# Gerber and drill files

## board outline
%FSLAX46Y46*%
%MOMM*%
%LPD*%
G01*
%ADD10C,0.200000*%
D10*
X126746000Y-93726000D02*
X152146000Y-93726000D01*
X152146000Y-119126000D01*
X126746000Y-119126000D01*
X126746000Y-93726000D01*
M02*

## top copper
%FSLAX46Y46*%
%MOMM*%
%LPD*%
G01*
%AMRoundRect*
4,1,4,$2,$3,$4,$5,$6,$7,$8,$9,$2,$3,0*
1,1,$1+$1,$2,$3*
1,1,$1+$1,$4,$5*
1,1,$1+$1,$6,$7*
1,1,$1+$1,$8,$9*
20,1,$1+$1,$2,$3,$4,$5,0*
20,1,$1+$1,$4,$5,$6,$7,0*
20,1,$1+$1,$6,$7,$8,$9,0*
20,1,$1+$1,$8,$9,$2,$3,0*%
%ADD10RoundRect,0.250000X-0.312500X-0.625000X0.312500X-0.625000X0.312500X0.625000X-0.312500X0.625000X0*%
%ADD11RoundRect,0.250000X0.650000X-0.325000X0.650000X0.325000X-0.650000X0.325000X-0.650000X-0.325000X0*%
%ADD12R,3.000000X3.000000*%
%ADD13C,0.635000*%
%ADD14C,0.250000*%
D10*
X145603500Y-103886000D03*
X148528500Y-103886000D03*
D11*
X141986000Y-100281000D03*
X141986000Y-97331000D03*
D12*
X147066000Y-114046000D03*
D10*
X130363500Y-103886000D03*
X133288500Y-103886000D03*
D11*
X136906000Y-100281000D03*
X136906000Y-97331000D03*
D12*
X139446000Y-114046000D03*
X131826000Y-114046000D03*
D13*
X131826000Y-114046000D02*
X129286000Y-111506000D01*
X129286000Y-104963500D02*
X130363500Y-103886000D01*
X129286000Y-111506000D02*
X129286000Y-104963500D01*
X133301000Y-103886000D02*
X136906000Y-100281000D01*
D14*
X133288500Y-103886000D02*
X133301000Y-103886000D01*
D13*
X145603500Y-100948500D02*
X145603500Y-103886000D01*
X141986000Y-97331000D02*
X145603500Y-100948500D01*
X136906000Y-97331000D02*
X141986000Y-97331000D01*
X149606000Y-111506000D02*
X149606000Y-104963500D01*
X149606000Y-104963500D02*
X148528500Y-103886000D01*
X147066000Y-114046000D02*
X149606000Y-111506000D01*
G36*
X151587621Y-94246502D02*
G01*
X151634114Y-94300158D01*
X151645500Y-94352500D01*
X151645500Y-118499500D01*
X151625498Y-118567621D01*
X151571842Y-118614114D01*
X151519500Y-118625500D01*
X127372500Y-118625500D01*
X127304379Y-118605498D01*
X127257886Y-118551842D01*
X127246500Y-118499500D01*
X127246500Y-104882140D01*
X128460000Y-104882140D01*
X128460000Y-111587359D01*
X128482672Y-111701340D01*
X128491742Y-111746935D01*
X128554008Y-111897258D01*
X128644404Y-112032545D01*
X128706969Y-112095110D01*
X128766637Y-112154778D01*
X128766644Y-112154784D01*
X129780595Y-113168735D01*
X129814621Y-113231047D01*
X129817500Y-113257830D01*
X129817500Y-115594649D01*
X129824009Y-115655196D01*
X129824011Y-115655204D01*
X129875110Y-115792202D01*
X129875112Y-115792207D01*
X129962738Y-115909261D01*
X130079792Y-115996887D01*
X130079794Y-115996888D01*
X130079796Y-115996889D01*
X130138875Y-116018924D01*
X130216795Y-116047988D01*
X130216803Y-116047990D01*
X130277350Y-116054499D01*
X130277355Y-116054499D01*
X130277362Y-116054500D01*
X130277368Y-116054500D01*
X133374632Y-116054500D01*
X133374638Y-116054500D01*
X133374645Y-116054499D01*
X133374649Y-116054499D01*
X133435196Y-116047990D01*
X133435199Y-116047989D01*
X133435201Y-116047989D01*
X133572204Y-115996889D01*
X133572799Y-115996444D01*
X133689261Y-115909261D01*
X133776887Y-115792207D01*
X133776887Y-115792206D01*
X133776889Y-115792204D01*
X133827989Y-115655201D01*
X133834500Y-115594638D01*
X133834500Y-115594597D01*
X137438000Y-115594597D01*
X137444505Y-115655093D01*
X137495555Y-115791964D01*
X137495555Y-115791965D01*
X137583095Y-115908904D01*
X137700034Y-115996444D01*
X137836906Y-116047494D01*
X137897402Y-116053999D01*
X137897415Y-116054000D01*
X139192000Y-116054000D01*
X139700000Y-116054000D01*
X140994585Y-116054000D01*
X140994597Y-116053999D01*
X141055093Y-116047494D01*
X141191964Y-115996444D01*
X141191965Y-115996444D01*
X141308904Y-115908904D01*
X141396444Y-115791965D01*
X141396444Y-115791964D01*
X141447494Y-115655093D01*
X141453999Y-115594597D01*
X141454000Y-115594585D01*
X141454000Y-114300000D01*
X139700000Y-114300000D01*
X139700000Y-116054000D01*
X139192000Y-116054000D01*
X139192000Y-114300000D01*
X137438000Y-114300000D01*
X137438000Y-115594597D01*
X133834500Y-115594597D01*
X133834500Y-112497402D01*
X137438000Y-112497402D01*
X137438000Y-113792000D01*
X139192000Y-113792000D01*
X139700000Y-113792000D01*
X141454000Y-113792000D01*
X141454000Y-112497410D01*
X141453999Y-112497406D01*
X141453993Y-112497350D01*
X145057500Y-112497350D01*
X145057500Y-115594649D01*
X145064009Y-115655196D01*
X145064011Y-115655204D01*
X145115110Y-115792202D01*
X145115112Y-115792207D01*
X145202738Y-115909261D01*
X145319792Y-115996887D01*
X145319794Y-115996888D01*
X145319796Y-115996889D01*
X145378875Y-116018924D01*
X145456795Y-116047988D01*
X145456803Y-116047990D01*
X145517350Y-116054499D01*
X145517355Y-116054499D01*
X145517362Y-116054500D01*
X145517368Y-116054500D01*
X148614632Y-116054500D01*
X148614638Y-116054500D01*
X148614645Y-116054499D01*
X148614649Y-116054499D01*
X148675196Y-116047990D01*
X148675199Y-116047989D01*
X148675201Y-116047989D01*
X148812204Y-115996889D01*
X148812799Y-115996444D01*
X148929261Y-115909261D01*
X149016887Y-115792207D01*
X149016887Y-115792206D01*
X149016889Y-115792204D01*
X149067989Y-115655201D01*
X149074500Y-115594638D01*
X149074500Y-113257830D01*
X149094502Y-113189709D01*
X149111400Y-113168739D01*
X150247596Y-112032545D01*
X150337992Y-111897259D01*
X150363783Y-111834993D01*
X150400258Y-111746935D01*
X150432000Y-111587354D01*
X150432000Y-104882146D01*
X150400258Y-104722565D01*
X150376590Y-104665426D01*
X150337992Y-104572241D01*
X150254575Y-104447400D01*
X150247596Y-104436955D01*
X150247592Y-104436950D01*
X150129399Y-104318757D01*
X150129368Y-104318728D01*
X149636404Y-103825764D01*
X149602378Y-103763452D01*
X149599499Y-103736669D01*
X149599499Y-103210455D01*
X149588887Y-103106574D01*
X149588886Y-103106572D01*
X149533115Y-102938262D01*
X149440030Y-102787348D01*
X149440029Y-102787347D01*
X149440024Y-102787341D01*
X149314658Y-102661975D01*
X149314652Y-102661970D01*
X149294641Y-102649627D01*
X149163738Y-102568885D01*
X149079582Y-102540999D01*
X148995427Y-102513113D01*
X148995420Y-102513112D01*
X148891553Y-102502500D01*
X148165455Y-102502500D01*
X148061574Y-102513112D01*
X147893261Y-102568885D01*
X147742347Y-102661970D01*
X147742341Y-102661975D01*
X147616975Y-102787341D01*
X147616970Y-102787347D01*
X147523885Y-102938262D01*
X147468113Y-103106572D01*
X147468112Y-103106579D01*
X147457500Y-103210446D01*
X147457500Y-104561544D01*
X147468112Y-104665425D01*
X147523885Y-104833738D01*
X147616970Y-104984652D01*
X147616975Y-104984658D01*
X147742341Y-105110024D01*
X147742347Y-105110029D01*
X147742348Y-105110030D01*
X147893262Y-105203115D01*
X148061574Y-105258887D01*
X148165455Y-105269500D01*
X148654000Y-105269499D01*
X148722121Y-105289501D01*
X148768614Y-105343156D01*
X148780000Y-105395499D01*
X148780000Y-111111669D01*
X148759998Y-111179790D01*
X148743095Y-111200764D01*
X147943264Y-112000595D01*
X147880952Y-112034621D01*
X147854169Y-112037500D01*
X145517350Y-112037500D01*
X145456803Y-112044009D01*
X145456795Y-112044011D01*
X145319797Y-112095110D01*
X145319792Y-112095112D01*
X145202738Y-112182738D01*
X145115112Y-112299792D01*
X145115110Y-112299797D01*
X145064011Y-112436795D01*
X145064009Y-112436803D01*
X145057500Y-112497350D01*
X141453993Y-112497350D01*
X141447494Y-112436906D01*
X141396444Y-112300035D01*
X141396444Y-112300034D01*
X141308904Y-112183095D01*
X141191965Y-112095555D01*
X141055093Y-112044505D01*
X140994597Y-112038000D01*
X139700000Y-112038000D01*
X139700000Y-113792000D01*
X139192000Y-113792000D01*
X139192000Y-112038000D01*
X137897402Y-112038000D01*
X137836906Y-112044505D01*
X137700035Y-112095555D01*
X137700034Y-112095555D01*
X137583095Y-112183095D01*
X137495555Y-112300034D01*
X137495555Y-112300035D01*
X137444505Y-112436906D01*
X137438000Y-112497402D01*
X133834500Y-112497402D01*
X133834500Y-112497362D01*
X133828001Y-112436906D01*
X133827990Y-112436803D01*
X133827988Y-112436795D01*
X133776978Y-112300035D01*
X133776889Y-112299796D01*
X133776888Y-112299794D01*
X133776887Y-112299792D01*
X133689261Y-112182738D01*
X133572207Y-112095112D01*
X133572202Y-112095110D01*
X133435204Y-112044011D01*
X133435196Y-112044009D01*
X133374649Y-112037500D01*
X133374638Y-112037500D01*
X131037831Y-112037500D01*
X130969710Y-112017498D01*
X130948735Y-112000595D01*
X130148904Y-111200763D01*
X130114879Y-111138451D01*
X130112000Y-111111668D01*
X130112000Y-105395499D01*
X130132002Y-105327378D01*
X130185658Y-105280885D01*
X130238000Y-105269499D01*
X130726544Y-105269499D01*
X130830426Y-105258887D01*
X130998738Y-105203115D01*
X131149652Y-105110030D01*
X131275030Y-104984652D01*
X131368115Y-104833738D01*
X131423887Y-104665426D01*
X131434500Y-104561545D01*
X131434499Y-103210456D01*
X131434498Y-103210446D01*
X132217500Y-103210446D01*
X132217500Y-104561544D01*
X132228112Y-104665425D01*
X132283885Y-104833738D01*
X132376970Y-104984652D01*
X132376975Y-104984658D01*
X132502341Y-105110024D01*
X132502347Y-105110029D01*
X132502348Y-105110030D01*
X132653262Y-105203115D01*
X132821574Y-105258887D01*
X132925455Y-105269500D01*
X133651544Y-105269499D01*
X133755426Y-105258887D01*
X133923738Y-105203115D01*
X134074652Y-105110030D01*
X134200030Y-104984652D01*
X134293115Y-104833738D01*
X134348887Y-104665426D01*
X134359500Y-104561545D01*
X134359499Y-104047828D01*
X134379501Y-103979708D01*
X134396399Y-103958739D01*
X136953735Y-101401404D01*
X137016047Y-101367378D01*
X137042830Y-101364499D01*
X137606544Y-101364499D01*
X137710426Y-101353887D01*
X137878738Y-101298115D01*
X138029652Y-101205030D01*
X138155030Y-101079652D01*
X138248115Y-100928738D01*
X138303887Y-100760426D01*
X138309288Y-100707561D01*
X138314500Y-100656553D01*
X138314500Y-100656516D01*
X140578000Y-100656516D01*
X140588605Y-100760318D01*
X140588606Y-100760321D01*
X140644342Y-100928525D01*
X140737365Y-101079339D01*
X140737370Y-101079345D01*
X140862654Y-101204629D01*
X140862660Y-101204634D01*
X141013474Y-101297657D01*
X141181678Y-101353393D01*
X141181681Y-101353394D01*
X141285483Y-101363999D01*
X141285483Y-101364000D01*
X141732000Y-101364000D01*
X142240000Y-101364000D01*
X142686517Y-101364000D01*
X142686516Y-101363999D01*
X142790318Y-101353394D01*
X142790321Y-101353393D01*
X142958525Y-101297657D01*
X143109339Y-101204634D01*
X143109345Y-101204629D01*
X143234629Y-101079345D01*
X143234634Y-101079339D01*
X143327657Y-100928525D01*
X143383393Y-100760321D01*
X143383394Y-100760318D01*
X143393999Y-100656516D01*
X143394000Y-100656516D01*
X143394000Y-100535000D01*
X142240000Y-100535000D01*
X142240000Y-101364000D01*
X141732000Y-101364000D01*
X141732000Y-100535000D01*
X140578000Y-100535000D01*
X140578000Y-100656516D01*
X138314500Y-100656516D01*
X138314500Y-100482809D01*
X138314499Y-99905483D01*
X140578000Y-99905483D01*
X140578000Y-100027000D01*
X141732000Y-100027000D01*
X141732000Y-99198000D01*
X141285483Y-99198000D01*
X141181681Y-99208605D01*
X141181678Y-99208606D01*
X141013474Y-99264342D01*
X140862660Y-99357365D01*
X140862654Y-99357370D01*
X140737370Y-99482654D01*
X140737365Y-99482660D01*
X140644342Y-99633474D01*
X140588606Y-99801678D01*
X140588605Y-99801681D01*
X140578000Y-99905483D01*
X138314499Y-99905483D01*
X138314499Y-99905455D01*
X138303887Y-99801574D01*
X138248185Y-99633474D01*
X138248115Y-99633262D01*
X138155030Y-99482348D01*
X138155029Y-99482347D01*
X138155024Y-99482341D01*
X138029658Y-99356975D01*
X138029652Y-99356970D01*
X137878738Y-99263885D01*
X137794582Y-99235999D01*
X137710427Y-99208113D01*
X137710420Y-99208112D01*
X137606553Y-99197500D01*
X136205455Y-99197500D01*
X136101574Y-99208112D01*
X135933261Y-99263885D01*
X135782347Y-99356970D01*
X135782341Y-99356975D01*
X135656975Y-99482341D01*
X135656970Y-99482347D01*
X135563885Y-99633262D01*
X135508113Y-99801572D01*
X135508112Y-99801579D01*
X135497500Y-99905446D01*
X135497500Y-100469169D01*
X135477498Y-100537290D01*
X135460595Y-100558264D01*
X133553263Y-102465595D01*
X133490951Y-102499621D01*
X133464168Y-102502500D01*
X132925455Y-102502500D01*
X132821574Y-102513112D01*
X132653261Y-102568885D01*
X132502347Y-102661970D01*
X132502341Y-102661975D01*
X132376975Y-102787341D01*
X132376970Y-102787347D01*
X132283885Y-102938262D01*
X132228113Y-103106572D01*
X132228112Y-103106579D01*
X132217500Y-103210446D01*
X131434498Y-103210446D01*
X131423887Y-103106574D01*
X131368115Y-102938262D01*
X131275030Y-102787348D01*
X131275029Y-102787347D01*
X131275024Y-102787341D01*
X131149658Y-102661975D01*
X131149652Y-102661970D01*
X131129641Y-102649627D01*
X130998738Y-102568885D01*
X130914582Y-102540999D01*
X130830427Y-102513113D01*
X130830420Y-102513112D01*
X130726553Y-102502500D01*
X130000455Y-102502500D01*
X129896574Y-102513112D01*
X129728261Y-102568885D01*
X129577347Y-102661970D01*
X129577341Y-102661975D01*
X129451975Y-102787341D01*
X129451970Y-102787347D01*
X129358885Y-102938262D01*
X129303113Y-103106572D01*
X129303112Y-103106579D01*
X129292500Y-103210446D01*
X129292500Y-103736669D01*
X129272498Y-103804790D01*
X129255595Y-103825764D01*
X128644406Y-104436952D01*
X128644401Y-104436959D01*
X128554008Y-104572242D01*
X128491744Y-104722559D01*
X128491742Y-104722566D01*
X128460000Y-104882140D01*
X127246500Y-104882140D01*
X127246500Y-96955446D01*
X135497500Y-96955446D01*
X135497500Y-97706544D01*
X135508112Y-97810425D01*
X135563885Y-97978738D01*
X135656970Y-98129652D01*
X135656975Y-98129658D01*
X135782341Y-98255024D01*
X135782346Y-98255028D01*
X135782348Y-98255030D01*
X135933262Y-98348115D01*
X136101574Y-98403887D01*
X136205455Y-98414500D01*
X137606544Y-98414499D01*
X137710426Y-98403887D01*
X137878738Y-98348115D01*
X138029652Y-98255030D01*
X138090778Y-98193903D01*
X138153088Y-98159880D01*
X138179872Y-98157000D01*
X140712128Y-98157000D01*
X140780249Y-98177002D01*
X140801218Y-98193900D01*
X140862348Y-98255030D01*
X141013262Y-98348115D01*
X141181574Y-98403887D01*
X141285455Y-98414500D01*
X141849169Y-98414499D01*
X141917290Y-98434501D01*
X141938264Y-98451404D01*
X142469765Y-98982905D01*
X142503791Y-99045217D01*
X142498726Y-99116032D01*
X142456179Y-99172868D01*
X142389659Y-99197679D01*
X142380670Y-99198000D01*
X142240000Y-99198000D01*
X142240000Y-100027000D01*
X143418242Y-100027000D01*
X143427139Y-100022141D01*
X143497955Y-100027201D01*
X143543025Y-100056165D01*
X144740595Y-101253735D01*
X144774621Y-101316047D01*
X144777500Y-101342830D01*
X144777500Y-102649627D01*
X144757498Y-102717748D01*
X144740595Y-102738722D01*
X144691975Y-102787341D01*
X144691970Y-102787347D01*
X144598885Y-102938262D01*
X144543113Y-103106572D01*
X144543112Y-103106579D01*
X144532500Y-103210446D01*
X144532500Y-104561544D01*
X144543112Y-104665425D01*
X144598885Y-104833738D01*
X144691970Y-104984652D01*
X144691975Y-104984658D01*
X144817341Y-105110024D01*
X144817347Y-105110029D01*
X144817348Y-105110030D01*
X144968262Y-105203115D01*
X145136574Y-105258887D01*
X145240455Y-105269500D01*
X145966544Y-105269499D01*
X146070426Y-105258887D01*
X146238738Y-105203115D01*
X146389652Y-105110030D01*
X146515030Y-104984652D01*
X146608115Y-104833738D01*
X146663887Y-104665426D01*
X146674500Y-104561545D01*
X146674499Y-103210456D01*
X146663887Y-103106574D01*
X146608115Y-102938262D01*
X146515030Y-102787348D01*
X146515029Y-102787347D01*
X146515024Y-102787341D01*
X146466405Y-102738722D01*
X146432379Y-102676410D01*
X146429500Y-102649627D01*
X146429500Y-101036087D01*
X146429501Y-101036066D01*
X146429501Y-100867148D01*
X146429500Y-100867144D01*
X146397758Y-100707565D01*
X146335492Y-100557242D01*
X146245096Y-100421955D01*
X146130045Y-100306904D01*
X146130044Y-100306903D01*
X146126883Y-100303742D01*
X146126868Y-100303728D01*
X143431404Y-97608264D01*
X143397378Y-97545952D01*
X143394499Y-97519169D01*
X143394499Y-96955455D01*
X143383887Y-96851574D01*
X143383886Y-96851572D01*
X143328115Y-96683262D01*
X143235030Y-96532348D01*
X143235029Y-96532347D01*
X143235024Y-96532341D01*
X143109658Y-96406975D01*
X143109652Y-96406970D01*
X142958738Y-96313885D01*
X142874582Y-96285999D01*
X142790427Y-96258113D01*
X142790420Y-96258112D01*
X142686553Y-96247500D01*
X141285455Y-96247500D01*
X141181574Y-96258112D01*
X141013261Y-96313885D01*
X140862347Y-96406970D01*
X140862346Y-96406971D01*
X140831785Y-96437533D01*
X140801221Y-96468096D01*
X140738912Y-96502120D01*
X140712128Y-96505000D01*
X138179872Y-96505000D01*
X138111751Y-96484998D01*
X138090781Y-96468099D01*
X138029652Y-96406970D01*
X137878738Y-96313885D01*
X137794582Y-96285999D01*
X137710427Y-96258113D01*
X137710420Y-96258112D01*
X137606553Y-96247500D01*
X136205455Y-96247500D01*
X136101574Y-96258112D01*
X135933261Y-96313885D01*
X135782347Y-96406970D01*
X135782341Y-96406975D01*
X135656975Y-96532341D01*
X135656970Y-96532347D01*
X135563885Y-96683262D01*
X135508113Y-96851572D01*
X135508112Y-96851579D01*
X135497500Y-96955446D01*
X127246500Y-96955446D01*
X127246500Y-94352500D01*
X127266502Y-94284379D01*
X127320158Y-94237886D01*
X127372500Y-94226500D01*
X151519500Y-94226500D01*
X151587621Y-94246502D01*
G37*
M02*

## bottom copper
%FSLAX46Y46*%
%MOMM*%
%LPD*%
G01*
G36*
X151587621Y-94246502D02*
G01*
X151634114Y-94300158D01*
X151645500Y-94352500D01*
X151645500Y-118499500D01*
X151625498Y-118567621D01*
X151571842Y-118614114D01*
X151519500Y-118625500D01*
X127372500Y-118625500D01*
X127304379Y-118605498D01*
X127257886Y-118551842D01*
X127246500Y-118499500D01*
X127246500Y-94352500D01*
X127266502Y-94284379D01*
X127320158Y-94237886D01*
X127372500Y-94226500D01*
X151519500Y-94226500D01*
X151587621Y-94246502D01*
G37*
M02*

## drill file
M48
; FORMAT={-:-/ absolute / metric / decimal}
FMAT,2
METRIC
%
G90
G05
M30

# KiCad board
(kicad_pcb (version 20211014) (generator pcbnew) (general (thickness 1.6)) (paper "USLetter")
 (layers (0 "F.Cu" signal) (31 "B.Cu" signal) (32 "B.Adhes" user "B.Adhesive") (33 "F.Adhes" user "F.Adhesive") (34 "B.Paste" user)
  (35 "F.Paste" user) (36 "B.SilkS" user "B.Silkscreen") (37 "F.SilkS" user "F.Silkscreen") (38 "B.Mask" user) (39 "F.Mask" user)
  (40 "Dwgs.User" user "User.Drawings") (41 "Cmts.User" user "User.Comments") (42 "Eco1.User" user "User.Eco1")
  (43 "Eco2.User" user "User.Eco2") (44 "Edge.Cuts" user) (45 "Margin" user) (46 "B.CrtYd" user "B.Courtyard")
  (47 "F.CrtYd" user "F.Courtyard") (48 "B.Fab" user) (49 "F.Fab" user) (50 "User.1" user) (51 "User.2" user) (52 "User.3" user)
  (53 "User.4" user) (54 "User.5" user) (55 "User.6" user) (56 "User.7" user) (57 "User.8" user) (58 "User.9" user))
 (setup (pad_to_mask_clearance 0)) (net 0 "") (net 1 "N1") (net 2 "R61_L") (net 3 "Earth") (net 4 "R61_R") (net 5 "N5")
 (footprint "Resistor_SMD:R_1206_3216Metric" (layer "F.Cu") (at 147.066 103.886)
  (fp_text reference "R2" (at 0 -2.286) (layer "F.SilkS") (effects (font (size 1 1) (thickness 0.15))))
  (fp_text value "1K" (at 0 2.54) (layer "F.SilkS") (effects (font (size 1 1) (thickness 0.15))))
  (pad "1" smd roundrect (at -1.4625 0) (size 1.125 1.75) (layers "F.Cu" "F.Paste" "F.Mask") (roundrect_rratio 0.2222222222) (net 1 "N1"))
  (pad "2" smd roundrect (at 1.4625 0) (size 1.125 1.75) (layers "F.Cu" "F.Paste" "F.Mask") (roundrect_rratio 0.2222222222) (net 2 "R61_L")))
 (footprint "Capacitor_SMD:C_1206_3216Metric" (layer "F.Cu") (at 141.986 98.806 90)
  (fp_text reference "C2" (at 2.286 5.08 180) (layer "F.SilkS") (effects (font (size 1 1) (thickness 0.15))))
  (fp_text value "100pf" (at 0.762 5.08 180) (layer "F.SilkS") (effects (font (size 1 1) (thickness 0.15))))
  (pad "1" smd roundrect (at -1.475 0 90) (size 1.15 1.8) (layers "F.Cu" "F.Paste" "F.Mask") (roundrect_rratio 0.2173913043) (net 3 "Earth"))
  (pad "2" smd roundrect (at 1.475 0 90) (size 1.15 1.8) (layers "F.Cu" "F.Paste" "F.Mask") (roundrect_rratio 0.2173913043) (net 1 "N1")))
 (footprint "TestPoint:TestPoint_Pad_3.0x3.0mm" (layer "F.Cu") (at 147.066 114.046)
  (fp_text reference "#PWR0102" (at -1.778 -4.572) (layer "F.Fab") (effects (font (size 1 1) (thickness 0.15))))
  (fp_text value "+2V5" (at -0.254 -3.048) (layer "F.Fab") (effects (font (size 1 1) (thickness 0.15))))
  (pad "1" smd rect (at 0 0) (size 3 3) (layers "F.Cu" "F.Paste" "F.Mask") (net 2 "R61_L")))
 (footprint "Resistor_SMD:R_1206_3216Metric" (layer "F.Cu") (at 131.826 103.886)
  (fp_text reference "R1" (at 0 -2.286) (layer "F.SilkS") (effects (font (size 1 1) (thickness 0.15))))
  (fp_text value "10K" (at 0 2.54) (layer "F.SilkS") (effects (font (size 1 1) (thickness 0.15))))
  (pad "1" smd roundrect (at -1.4625 0) (size 1.125 1.75) (layers "F.Cu" "F.Paste" "F.Mask") (roundrect_rratio 0.2222222222) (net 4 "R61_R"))
  (pad "2" smd roundrect (at 1.4625 0) (size 1.125 1.75) (layers "F.Cu" "F.Paste" "F.Mask") (roundrect_rratio 0.2222222222) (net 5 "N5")))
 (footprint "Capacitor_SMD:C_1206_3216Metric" (layer "F.Cu") (at 136.906 98.806 90)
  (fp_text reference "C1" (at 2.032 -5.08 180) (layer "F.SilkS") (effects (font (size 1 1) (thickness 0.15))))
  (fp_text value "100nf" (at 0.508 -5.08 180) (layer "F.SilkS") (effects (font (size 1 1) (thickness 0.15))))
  (pad "1" smd roundrect (at -1.475 0 90) (size 1.15 1.8) (layers "F.Cu" "F.Paste" "F.Mask") (roundrect_rratio 0.2173913043) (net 5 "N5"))
  (pad "2" smd roundrect (at 1.475 0 90) (size 1.15 1.8) (layers "F.Cu" "F.Paste" "F.Mask") (roundrect_rratio 0.2173913043) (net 1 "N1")))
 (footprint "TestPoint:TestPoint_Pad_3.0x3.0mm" (layer "F.Cu") (at 139.446 114.046)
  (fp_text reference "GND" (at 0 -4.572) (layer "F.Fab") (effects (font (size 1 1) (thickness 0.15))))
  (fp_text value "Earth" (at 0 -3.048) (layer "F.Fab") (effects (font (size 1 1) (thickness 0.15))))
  (pad "1" smd rect (at 0 0) (size 3 3) (layers "F.Cu" "F.Paste" "F.Mask") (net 3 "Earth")))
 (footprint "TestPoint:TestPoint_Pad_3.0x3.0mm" (layer "F.Cu") (at 131.826 114.046)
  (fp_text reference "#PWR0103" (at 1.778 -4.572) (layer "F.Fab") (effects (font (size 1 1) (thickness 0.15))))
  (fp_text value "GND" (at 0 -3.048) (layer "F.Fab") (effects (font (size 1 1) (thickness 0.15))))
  (pad "1" smd rect (at 0 0) (size 3 3) (layers "F.Cu" "F.Paste" "F.Mask") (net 4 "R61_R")))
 (gr_rect (start 126.746 93.726) (end 152.146 119.126) (layer "Edge.Cuts") (width 0.2) (fill none))
 (segment (start 131.826 114.046) (end 129.286 111.506) (width 0.635) (layer "F.Cu") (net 4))
 (segment (start 129.286 104.9635) (end 130.3635 103.886) (width 0.635) (layer "F.Cu") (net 4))
 (segment (start 129.286 111.506) (end 129.286 104.9635) (width 0.635) (layer "F.Cu") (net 4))
 (segment (start 133.301 103.886) (end 136.906 100.281) (width 0.635) (layer "F.Cu") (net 5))
 (segment (start 133.2885 103.886) (end 133.301 103.886) (width 0.25) (layer "F.Cu") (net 5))
 (segment (start 145.6035 100.9485) (end 145.6035 103.886) (width 0.635) (layer "F.Cu") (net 1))
 (segment (start 141.986 97.331) (end 145.6035 100.9485) (width 0.635) (layer "F.Cu") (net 1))
 (segment (start 136.906 97.331) (end 141.986 97.331) (width 0.635) (layer "F.Cu") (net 1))
 (segment (start 149.606 111.506) (end 149.606 104.9635) (width 0.635) (layer "F.Cu") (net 2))
 (segment (start 149.606 104.9635) (end 148.5285 103.886) (width 0.635) (layer "F.Cu") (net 2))
 (segment (start 147.066 114.046) (end 149.606 111.506) (width 0.635) (layer "F.Cu") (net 2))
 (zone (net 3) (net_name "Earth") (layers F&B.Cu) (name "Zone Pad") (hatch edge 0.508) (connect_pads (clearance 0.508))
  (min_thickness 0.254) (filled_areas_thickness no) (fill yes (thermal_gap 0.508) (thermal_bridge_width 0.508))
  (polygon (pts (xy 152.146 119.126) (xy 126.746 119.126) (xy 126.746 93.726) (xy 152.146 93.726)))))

